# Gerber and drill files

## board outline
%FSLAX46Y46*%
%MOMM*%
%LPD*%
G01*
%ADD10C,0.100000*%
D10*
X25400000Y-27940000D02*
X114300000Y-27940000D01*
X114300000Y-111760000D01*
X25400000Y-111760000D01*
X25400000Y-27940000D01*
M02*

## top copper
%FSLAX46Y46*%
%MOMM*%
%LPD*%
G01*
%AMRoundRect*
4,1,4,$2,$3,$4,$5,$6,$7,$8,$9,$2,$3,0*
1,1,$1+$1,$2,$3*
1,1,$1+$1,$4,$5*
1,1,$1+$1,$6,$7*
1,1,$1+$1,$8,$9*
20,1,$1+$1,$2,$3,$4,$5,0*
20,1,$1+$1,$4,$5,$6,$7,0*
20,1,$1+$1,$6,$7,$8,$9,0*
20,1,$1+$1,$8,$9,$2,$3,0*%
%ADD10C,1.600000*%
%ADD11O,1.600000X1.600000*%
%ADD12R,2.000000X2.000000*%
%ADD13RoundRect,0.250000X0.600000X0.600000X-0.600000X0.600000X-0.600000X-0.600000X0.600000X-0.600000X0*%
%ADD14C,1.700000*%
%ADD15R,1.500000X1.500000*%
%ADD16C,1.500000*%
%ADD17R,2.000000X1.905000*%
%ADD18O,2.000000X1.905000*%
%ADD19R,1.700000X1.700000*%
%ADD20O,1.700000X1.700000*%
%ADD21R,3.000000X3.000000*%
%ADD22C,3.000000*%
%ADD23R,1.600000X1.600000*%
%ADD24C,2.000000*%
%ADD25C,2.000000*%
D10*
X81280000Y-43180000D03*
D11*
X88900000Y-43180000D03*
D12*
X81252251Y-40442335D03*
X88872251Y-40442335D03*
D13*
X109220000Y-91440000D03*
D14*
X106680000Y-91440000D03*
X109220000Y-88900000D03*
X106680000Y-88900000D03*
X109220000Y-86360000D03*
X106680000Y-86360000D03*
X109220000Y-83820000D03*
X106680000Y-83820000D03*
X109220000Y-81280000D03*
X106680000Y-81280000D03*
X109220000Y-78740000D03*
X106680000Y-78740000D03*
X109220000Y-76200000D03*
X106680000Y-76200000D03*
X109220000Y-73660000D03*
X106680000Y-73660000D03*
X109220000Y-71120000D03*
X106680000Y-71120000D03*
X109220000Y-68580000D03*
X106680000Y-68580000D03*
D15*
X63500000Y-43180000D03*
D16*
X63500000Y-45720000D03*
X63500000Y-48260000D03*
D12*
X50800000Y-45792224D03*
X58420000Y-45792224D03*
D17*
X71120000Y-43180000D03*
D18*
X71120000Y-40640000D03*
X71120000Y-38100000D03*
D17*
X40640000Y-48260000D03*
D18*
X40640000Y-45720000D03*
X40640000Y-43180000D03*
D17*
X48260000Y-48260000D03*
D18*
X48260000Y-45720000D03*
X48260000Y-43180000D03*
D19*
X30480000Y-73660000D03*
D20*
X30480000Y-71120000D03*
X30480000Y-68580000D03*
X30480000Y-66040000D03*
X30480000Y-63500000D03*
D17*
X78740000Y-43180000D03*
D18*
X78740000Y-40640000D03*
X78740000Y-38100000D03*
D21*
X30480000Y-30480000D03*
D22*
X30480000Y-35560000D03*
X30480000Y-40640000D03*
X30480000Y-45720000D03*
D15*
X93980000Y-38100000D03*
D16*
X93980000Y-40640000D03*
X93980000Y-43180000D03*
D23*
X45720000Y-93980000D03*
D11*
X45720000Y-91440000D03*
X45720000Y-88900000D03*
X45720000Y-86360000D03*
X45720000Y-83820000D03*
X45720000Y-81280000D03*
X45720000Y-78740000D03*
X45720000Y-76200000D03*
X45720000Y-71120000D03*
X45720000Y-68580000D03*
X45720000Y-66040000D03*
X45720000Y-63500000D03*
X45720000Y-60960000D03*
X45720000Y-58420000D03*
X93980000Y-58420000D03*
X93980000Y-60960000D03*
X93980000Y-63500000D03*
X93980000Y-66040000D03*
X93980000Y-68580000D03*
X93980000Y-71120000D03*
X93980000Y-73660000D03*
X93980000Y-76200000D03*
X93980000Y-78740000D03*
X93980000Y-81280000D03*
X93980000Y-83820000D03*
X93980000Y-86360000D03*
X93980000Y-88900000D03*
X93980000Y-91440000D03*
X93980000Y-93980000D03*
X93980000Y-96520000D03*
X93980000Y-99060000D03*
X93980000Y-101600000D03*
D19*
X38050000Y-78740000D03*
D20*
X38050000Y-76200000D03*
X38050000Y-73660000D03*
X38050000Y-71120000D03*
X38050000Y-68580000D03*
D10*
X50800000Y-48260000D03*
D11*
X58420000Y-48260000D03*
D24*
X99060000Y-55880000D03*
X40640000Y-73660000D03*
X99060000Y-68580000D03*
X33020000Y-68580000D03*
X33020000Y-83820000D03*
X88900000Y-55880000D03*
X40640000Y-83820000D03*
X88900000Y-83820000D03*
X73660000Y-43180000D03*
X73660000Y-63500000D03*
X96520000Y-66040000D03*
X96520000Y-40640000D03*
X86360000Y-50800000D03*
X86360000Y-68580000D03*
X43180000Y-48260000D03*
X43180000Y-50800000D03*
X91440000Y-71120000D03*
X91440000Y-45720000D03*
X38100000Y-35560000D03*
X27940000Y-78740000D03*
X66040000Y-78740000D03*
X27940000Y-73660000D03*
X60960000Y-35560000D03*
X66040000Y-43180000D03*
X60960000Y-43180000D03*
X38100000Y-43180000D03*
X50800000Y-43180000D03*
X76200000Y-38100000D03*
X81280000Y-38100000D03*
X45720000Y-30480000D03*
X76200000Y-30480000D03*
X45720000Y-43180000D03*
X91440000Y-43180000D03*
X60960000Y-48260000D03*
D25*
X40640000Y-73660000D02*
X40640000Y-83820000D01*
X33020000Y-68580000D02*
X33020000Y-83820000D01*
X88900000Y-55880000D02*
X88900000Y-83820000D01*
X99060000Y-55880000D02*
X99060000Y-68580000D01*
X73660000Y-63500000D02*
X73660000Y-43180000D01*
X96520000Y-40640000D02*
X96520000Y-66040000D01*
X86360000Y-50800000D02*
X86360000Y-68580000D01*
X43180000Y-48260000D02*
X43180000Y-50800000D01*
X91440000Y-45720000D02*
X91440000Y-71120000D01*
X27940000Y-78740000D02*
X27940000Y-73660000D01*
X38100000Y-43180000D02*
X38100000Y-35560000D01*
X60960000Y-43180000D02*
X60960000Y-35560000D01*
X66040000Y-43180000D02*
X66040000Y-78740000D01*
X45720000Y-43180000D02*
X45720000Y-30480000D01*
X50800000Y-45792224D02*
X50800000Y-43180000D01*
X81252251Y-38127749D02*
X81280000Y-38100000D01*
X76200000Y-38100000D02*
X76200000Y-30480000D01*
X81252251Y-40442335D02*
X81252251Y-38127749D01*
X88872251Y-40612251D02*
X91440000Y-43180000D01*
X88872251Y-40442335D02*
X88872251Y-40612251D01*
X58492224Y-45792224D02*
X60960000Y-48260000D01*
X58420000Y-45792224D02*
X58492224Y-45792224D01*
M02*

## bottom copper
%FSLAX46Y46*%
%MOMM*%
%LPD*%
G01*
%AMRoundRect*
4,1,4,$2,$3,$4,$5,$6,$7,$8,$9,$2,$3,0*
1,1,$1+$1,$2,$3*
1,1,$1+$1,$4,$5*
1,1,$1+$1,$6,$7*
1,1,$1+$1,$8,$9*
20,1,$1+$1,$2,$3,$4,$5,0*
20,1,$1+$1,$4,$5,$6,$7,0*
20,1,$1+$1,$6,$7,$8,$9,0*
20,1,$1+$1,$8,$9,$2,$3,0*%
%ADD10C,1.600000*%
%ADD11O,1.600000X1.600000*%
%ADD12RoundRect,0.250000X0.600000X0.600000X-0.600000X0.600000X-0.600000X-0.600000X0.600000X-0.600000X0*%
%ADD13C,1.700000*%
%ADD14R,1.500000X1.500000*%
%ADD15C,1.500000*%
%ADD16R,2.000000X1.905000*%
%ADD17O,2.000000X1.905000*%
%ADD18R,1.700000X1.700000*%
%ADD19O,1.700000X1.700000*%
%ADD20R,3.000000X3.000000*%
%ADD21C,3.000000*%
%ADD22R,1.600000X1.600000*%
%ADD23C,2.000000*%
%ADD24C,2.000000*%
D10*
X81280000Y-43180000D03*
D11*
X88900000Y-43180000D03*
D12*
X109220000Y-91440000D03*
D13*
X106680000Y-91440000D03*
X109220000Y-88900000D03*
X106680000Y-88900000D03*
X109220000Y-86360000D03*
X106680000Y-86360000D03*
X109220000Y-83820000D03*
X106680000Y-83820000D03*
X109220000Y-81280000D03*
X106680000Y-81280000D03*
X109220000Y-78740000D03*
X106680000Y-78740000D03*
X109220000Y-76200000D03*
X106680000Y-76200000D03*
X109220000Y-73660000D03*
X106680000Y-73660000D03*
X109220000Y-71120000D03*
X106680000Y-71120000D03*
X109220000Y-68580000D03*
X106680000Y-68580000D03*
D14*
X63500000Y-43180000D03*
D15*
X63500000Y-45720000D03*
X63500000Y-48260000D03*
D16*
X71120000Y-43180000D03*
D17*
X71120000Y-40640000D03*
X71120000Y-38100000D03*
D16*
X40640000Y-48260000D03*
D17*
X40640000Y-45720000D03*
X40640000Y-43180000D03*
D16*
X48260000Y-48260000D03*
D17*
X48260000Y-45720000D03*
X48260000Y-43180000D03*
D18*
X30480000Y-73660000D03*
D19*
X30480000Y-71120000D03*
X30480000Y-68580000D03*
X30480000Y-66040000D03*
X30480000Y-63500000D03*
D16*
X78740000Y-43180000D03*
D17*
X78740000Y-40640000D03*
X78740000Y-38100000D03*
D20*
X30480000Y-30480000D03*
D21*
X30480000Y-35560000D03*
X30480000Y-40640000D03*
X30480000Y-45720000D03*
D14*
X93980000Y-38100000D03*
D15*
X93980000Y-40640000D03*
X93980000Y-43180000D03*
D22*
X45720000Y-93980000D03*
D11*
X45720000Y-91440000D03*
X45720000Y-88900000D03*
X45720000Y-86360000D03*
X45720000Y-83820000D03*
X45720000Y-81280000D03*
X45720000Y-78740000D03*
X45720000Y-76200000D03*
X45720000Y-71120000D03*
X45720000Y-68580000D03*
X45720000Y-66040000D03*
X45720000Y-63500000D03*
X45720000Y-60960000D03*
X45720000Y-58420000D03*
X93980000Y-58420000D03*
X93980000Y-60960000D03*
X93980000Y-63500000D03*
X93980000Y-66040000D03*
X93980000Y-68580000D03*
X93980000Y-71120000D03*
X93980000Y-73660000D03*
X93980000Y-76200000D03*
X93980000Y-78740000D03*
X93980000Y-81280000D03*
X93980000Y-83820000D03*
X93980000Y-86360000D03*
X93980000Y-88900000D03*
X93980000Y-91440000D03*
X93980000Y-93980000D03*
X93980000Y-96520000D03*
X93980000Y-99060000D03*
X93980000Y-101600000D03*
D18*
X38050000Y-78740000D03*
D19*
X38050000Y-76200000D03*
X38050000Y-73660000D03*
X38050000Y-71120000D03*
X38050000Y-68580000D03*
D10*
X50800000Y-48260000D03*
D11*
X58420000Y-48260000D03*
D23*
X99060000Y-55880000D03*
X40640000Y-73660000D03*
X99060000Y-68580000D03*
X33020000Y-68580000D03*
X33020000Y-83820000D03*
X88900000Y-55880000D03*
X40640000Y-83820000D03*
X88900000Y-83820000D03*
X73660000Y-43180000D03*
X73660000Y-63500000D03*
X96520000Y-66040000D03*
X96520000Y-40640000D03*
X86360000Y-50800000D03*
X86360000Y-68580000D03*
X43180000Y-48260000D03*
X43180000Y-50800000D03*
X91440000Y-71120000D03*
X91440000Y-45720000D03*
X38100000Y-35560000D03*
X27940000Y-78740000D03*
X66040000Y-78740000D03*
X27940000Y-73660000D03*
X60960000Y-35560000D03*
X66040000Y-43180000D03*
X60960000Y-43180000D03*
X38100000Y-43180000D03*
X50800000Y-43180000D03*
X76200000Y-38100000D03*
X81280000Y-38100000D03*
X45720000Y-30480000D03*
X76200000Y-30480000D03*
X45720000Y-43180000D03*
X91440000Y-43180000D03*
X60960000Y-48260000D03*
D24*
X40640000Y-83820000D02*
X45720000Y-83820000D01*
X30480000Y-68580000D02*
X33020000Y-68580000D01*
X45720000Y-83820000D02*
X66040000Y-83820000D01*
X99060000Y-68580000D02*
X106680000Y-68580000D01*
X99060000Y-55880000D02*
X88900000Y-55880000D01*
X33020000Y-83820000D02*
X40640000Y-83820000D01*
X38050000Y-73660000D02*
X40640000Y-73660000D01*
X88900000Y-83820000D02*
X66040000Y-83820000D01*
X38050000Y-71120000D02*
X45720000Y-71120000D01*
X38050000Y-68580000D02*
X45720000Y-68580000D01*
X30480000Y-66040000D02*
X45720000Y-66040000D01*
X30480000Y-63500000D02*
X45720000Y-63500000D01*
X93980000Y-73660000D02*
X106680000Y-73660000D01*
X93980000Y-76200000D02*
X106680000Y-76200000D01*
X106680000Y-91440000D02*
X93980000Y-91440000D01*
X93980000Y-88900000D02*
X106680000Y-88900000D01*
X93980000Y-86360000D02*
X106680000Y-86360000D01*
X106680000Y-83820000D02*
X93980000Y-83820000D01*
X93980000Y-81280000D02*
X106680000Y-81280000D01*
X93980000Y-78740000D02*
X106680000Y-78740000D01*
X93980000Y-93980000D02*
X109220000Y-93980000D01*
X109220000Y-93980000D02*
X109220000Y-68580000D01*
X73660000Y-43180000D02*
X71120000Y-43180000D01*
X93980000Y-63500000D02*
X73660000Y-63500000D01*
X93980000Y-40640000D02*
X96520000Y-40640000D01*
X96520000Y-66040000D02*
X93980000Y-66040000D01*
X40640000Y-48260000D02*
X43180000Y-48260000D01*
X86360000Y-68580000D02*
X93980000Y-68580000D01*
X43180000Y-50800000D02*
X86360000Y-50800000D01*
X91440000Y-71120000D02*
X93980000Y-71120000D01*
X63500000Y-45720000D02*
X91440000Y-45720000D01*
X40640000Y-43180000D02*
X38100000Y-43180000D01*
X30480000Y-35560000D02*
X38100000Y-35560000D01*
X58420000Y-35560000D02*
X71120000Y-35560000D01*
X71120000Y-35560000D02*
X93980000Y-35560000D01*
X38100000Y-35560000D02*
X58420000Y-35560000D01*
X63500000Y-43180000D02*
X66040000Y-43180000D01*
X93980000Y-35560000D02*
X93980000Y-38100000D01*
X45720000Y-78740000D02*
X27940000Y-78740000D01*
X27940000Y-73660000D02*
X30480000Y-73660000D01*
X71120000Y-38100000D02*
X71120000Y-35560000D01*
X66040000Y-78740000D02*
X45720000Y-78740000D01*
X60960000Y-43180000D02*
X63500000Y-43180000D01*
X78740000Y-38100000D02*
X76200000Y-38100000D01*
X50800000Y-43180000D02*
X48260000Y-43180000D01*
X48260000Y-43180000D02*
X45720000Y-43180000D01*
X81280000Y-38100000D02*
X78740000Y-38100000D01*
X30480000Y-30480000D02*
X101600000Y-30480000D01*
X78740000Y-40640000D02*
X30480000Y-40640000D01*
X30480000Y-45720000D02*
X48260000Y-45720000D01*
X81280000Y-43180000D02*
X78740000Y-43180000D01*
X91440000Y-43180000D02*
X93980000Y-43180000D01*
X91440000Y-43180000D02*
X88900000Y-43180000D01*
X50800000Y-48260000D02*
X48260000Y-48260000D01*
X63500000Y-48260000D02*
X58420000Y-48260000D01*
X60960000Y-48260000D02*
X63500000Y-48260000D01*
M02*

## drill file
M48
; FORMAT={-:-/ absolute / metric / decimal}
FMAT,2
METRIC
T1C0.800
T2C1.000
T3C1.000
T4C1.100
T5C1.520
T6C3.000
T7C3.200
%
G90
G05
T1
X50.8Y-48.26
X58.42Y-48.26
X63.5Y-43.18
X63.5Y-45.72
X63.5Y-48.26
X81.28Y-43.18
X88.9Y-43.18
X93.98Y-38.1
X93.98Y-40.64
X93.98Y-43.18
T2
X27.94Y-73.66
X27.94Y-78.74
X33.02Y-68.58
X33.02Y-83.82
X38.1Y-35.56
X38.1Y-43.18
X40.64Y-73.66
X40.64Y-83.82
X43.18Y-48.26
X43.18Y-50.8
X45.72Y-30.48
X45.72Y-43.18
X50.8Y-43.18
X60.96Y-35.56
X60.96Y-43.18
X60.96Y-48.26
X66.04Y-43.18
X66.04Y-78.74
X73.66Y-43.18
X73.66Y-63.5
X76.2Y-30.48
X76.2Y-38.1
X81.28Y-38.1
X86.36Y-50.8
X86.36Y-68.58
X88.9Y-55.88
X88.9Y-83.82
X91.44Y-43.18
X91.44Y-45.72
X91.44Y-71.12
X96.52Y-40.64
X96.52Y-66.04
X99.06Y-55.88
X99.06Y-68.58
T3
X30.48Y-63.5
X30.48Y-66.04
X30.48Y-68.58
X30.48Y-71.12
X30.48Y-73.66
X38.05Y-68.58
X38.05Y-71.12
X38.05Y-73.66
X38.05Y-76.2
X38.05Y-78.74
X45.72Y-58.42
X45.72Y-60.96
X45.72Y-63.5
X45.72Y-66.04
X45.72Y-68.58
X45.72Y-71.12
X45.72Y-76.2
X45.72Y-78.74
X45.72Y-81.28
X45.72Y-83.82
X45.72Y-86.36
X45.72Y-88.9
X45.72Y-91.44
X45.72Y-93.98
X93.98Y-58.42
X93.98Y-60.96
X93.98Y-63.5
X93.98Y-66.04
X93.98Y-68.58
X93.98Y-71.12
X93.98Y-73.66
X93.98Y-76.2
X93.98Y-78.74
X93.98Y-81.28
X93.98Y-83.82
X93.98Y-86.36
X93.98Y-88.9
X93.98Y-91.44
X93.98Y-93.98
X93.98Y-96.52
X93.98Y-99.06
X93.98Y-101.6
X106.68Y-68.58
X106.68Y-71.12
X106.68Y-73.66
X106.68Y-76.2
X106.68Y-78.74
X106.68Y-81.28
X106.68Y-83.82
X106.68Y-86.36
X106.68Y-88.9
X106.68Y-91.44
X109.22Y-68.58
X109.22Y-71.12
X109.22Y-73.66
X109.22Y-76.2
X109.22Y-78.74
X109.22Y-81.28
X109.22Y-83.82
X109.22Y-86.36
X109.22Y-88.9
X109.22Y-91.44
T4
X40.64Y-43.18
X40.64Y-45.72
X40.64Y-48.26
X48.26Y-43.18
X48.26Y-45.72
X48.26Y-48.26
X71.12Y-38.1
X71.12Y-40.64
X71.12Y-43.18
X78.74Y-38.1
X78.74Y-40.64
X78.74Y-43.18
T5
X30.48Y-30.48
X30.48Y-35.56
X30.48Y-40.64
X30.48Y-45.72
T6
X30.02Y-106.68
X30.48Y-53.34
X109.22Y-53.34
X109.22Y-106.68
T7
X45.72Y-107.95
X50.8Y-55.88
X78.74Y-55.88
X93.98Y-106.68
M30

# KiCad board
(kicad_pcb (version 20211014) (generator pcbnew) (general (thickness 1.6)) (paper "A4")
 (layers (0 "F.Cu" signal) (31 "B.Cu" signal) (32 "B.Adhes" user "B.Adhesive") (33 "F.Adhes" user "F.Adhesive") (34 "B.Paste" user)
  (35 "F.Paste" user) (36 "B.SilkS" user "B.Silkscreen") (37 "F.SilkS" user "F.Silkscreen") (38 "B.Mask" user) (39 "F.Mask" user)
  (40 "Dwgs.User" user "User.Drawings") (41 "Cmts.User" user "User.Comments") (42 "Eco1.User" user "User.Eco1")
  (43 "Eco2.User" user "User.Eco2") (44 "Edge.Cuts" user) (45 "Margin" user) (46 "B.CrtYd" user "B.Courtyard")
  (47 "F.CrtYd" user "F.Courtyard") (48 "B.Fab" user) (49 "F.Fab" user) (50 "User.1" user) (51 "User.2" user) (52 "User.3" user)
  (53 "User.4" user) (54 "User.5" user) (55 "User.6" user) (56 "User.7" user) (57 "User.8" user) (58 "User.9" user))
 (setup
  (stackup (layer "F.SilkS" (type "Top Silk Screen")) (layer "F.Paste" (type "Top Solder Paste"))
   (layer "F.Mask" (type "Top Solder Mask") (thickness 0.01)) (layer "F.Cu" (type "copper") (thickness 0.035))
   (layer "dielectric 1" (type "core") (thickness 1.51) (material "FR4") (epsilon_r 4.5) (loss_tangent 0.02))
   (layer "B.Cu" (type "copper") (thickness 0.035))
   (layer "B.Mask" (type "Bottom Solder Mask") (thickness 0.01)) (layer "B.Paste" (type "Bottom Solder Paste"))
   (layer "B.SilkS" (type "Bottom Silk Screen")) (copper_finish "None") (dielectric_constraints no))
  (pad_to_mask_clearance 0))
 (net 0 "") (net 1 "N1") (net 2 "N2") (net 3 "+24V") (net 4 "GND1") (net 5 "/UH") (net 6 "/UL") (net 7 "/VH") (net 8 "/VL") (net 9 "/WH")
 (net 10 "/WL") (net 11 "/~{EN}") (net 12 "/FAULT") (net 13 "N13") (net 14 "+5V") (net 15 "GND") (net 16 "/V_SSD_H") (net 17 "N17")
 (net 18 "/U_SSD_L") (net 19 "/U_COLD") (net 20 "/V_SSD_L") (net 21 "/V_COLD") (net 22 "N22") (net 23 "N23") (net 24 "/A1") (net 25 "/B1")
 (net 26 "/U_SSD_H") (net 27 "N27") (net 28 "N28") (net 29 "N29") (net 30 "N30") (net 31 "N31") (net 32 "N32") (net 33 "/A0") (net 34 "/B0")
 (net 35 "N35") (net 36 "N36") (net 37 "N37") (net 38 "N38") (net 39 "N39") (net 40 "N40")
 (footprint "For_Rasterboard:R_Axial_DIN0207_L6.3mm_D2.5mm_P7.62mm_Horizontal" (layer "F.Cu") (at 81.28 43.18)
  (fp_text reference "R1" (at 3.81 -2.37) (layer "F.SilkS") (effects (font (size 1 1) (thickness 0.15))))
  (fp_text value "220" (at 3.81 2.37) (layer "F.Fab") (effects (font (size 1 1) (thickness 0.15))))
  (pad "1" thru_hole circle (at 0 0) (size 1.6 1.6) (drill 0.8) (layers *.Cu *.Mask) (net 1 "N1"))
  (pad "2" thru_hole oval (at 7.62 0) (size 1.6 1.6) (drill 0.8) (layers *.Cu *.Mask) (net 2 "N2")))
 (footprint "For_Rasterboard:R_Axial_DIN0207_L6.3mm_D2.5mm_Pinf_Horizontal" (layer "F.Cu") (at 81.252251 40.442335)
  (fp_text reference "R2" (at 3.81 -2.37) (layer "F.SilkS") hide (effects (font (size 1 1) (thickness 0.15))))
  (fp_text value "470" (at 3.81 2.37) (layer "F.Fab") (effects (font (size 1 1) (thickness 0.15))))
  (pad "1" smd rect locked (at 0 0) (size 2 2) (layers "F.Cu") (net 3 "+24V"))
  (pad "2" smd rect locked (at 7.62 0) (size 2 2) (layers "F.Cu") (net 2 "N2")))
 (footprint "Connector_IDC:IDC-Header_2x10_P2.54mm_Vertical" (layer "F.Cu") (at 109.22 91.44 180)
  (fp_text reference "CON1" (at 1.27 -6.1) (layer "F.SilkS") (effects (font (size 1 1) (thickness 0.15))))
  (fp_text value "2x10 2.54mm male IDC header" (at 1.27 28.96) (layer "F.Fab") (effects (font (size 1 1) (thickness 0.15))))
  (pad "1" thru_hole roundrect (at 0 0 180) (size 1.7 1.7) (drill 1) (layers *.Cu *.Mask) (roundrect_rratio 0.147059) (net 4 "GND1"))
  (pad "2" thru_hole circle (at 2.54 0 180) (size 1.7 1.7) (drill 1) (layers *.Cu *.Mask) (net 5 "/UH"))
  (pad "3" thru_hole circle (at 0 2.54 180) (size 1.7 1.7) (drill 1) (layers *.Cu *.Mask) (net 4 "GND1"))
  (pad "4" thru_hole circle (at 2.54 2.54 180) (size 1.7 1.7) (drill 1) (layers *.Cu *.Mask) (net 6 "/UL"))
  (pad "5" thru_hole circle (at 0 5.08 180) (size 1.7 1.7) (drill 1) (layers *.Cu *.Mask) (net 4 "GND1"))
  (pad "6" thru_hole circle (at 2.54 5.08 180) (size 1.7 1.7) (drill 1) (layers *.Cu *.Mask) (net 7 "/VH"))
  (pad "7" thru_hole circle (at 0 7.62 180) (size 1.7 1.7) (drill 1) (layers *.Cu *.Mask) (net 4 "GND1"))
  (pad "8" thru_hole circle (at 2.54 7.62 180) (size 1.7 1.7) (drill 1) (layers *.Cu *.Mask) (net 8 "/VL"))
  (pad "9" thru_hole circle (at 0 10.16 180) (size 1.7 1.7) (drill 1) (layers *.Cu *.Mask) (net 4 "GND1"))
  (pad "10" thru_hole circle (at 2.54 10.16 180) (size 1.7 1.7) (drill 1) (layers *.Cu *.Mask) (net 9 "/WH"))
  (pad "11" thru_hole circle (at 0 12.7 180) (size 1.7 1.7) (drill 1) (layers *.Cu *.Mask) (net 4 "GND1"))
  (pad "12" thru_hole circle (at 2.54 12.7 180) (size 1.7 1.7) (drill 1) (layers *.Cu *.Mask) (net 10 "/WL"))
  (pad "13" thru_hole circle (at 0 15.24 180) (size 1.7 1.7) (drill 1) (layers *.Cu *.Mask) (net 4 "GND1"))
  (pad "14" thru_hole circle (at 2.54 15.24 180) (size 1.7 1.7) (drill 1) (layers *.Cu *.Mask) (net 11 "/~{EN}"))
  (pad "15" thru_hole circle (at 0 17.78 180) (size 1.7 1.7) (drill 1) (layers *.Cu *.Mask) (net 4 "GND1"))
  (pad "16" thru_hole circle (at 2.54 17.78 180) (size 1.7 1.7) (drill 1) (layers *.Cu *.Mask) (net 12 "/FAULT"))
  (pad "17" thru_hole circle (at 0 20.32 180) (size 1.7 1.7) (drill 1) (layers *.Cu *.Mask) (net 4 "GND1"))
  (pad "18" thru_hole circle (at 2.54 20.32 180) (size 1.7 1.7) (drill 1) (layers *.Cu *.Mask) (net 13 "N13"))
  (pad "19" thru_hole circle (at 0 22.86 180) (size 1.7 1.7) (drill 1) (layers *.Cu *.Mask) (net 4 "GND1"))
  (pad "20" thru_hole circle (at 2.54 22.86 180) (size 1.7 1.7) (drill 1) (layers *.Cu *.Mask) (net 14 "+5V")))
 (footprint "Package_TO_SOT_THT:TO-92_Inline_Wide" (layer "F.Cu") (at 63.5 43.18 -90)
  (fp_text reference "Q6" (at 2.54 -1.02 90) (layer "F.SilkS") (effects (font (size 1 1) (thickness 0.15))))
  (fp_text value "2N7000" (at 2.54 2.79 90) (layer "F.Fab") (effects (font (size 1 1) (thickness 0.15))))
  (pad "1" thru_hole rect (at 0 0 270) (size 1.5 1.5) (drill 0.8) (layers *.Cu *.Mask) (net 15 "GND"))
  (pad "2" thru_hole circle (at 2.54 0 270) (size 1.5 1.5) (drill 0.8) (layers *.Cu *.Mask) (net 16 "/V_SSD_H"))
  (pad "3" thru_hole circle (at 5.08 0 270) (size 1.5 1.5) (drill 0.8) (layers *.Cu *.Mask) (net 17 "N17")))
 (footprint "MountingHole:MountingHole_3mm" (layer "F.Cu") (at 30.02 106.68)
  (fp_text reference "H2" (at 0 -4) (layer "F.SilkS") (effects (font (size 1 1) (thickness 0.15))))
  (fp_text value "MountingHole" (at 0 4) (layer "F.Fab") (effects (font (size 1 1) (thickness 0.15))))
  (pad "" np_thru_hole circle (at 0 0) (size 3 3) (drill 3) (layers *.Cu *.Mask)))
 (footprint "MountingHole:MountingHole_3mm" (layer "F.Cu") (at 109.22 53.34)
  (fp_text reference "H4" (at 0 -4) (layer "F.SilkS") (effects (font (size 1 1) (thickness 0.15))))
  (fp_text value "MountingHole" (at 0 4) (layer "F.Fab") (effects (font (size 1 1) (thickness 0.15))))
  (pad "" np_thru_hole circle (at 0 0) (size 3 3) (drill 3) (layers *.Cu *.Mask)))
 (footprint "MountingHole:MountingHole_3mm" (layer "F.Cu") (at 109.22 106.68)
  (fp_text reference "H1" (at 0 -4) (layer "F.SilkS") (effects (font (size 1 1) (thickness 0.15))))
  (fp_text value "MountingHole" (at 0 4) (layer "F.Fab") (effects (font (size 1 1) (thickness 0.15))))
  (pad "" np_thru_hole circle (at 0 0) (size 3 3) (drill 3) (layers *.Cu *.Mask)))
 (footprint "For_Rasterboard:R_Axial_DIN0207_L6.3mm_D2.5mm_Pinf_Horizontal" (layer "F.Cu") (at 50.8 45.792224)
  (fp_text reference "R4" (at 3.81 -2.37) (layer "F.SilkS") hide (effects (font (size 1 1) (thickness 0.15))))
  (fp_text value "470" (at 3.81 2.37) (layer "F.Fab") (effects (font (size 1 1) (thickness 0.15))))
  (pad "1" smd rect locked (at 0 0) (size 2 2) (layers "F.Cu") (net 3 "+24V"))
  (pad "2" smd rect locked (at 7.62 0) (size 2 2) (layers "F.Cu") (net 17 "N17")))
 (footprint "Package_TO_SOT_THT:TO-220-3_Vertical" (layer "F.Cu") (at 71.12 43.18 90)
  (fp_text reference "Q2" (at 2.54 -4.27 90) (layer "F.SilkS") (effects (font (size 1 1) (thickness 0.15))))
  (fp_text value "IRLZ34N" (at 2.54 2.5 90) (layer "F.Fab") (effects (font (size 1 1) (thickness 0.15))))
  (pad "1" thru_hole rect (at 0 0 90) (size 1.905 2) (drill 1.1) (layers *.Cu *.Mask) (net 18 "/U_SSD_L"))
  (pad "2" thru_hole oval (at 2.54 0 90) (size 1.905 2) (drill 1.1) (layers *.Cu *.Mask) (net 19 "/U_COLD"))
  (pad "3" thru_hole oval (at 5.08 0 90) (size 1.905 2) (drill 1.1) (layers *.Cu *.Mask) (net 15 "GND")))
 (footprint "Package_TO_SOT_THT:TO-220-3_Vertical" (layer "F.Cu") (at 40.64 48.26 90)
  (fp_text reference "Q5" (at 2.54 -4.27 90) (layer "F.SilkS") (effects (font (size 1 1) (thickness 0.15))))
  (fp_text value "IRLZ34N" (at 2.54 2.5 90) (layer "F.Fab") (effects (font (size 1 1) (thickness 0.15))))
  (pad "1" thru_hole rect (at 0 0 90) (size 1.905 2) (drill 1.1) (layers *.Cu *.Mask) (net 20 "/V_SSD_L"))
  (pad "2" thru_hole oval (at 2.54 0 90) (size 1.905 2) (drill 1.1) (layers *.Cu *.Mask) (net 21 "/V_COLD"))
  (pad "3" thru_hole oval (at 5.08 0 90) (size 1.905 2) (drill 1.1) (layers *.Cu *.Mask) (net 15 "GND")))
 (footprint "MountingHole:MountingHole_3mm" (layer "F.Cu") (at 30.48 53.34)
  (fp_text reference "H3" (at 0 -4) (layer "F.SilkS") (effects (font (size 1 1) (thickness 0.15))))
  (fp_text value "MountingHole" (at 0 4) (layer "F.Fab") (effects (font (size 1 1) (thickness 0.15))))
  (pad "" np_thru_hole circle (at 0 0) (size 3 3) (drill 3) (layers *.Cu *.Mask)))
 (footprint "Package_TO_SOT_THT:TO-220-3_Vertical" (layer "F.Cu") (at 48.26 48.26 90)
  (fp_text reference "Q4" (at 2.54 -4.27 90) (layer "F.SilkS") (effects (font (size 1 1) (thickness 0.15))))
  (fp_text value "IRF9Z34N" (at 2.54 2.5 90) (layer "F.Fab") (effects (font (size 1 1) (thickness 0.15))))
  (pad "1" thru_hole rect (at 0 0 90) (size 1.905 2) (drill 1.1) (layers *.Cu *.Mask) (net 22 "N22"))
  (pad "2" thru_hole oval (at 2.54 0 90) (size 1.905 2) (drill 1.1) (layers *.Cu *.Mask) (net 21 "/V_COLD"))
  (pad "3" thru_hole oval (at 5.08 0 90) (size 1.905 2) (drill 1.1) (layers *.Cu *.Mask) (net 3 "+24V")))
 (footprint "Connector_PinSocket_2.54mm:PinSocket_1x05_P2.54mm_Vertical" (layer "F.Cu") (at 30.48 73.66 180)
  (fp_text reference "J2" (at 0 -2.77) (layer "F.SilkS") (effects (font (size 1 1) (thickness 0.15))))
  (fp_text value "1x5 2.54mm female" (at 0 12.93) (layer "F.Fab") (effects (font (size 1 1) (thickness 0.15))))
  (pad "1" thru_hole rect (at 0 0 180) (size 1.7 1.7) (drill 1) (layers *.Cu *.Mask) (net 15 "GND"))
  (pad "2" thru_hole oval (at 0 2.54 180) (size 1.7 1.7) (drill 1) (layers *.Cu *.Mask) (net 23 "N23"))
  (pad "3" thru_hole oval (at 0 5.08 180) (size 1.7 1.7) (drill 1) (layers *.Cu *.Mask) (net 14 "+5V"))
  (pad "4" thru_hole oval (at 0 7.62 180) (size 1.7 1.7) (drill 1) (layers *.Cu *.Mask) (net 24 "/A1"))
  (pad "5" thru_hole oval (at 0 10.16 180) (size 1.7 1.7) (drill 1) (layers *.Cu *.Mask) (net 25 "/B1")))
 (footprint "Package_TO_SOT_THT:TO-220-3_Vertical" (layer "F.Cu") (at 78.74 43.18 90)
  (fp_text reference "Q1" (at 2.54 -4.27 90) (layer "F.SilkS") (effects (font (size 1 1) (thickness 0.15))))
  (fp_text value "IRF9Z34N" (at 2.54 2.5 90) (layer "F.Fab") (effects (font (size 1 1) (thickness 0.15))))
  (pad "1" thru_hole rect (at 0 0 90) (size 1.905 2) (drill 1.1) (layers *.Cu *.Mask) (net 1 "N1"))
  (pad "2" thru_hole oval (at 2.54 0 90) (size 1.905 2) (drill 1.1) (layers *.Cu *.Mask) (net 19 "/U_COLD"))
  (pad "3" thru_hole oval (at 5.08 0 90) (size 1.905 2) (drill 1.1) (layers *.Cu *.Mask) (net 3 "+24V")))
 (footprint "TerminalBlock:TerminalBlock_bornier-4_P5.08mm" (layer "F.Cu") (at 30.48 30.48 -90)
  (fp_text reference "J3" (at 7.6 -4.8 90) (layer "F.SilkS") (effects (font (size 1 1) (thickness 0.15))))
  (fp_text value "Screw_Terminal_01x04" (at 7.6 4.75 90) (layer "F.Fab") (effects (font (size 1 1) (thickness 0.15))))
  (pad "1" thru_hole rect (at 0 0 270) (size 3 3) (drill 1.52) (layers *.Cu *.Mask) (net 3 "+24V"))
  (pad "2" thru_hole circle (at 5.08 0 270) (size 3 3) (drill 1.52) (layers *.Cu *.Mask) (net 15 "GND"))
  (pad "3" thru_hole circle (at 10.16 0 270) (size 3 3) (drill 1.52) (layers *.Cu *.Mask) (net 19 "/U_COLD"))
  (pad "4" thru_hole circle (at 15.24 0 270) (size 3 3) (drill 1.52) (layers *.Cu *.Mask) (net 21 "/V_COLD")))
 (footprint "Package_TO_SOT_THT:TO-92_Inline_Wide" (layer "F.Cu") (at 93.98 38.1 -90)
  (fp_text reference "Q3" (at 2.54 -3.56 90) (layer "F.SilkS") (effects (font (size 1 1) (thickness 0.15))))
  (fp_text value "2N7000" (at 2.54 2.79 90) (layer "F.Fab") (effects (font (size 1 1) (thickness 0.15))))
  (pad "1" thru_hole rect (at 0 0 270) (size 1.5 1.5) (drill 0.8) (layers *.Cu *.Mask) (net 15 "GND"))
  (pad "2" thru_hole circle (at 2.54 0 270) (size 1.5 1.5) (drill 0.8) (layers *.Cu *.Mask) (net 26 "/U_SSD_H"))
  (pad "3" thru_hole circle (at 5.08 0 270) (size 1.5 1.5) (drill 0.8) (layers *.Cu *.Mask) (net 2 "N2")))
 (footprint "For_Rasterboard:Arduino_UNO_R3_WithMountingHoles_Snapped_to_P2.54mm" (layer "F.Cu") (at 45.72 93.98 90)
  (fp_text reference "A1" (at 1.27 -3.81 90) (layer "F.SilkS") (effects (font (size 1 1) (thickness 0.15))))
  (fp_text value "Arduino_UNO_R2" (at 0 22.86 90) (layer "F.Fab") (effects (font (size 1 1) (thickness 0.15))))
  (pad "" np_thru_hole circle (at -13.97 0 180) (size 3.2 3.2) (drill 3.2) (layers *.Cu *.Mask))
  (pad "" np_thru_hole circle (at 38.1 5.08 180) (size 3.2 3.2) (drill 3.2) (layers *.Cu *.Mask))
  (pad "" np_thru_hole circle (at -12.7 48.26 180) (size 3.2 3.2) (drill 3.2) (layers *.Cu *.Mask))
  (pad "" np_thru_hole circle (at 38.1 33.02 180) (size 3.2 3.2) (drill 3.2) (layers *.Cu *.Mask))
  (pad "1" thru_hole rect (at 0 0 180) (size 1.6 1.6) (drill 1) (layers *.Cu *.Mask) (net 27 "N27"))
  (pad "2" thru_hole oval (at 2.54 0 180) (size 1.6 1.6) (drill 1) (layers *.Cu *.Mask) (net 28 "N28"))
  (pad "3" thru_hole oval (at 5.08 0 180) (size 1.6 1.6) (drill 1) (layers *.Cu *.Mask) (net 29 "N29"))
  (pad "4" thru_hole oval (at 7.62 0 180) (size 1.6 1.6) (drill 1) (layers *.Cu *.Mask) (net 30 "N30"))
  (pad "5" thru_hole oval (at 10.16 0 180) (size 1.6 1.6) (drill 1) (layers *.Cu *.Mask) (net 14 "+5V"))
  (pad "6" thru_hole oval (at 12.7 0 180) (size 1.6 1.6) (drill 1) (layers *.Cu *.Mask) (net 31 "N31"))
  (pad "7" thru_hole oval (at 15.24 0 180) (size 1.6 1.6) (drill 1) (layers *.Cu *.Mask) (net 15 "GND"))
  (pad "8" thru_hole oval (at 17.78 0 180) (size 1.6 1.6) (drill 1) (layers *.Cu *.Mask) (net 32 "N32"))
  (pad "9" thru_hole oval (at 22.86 0 180) (size 1.6 1.6) (drill 1) (layers *.Cu *.Mask) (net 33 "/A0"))
  (pad "10" thru_hole oval (at 25.4 0 180) (size 1.6 1.6) (drill 1) (layers *.Cu *.Mask) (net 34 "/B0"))
  (pad "11" thru_hole oval (at 27.94 0 180) (size 1.6 1.6) (drill 1) (layers *.Cu *.Mask) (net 24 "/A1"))
  (pad "12" thru_hole oval (at 30.48 0 180) (size 1.6 1.6) (drill 1) (layers *.Cu *.Mask) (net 25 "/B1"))
  (pad "13" thru_hole oval (at 33.02 0 180) (size 1.6 1.6) (drill 1) (layers *.Cu *.Mask) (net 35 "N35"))
  (pad "14" thru_hole oval (at 35.56 0 180) (size 1.6 1.6) (drill 1) (layers *.Cu *.Mask) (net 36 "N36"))
  (pad "15" thru_hole oval (at 35.56 48.26 180) (size 1.6 1.6) (drill 1) (layers *.Cu *.Mask) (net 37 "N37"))
  (pad "16" thru_hole oval (at 33.02 48.26 180) (size 1.6 1.6) (drill 1) (layers *.Cu *.Mask) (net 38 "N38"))
  (pad "17" thru_hole oval (at 30.48 48.26 180) (size 1.6 1.6) (drill 1) (layers *.Cu *.Mask) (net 18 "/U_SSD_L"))
  (pad "18" thru_hole oval (at 27.94 48.26 180) (size 1.6 1.6) (drill 1) (layers *.Cu *.Mask) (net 26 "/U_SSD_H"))
  (pad "19" thru_hole oval (at 25.4 48.26 180) (size 1.6 1.6) (drill 1) (layers *.Cu *.Mask) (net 20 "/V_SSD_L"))
  (pad "20" thru_hole oval (at 22.86 48.26 180) (size 1.6 1.6) (drill 1) (layers *.Cu *.Mask) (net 16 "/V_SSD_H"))
  (pad "21" thru_hole oval (at 20.32 48.26 180) (size 1.6 1.6) (drill 1) (layers *.Cu *.Mask) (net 12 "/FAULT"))
  (pad "22" thru_hole oval (at 17.78 48.26 180) (size 1.6 1.6) (drill 1) (layers *.Cu *.Mask) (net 11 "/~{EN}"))
  (pad "23" thru_hole oval (at 15.24 48.26 180) (size 1.6 1.6) (drill 1) (layers *.Cu *.Mask) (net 10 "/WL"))
  (pad "24" thru_hole oval (at 12.7 48.26 180) (size 1.6 1.6) (drill 1) (layers *.Cu *.Mask) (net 9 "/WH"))
  (pad "25" thru_hole oval (at 10.16 48.26 180) (size 1.6 1.6) (drill 1) (layers *.Cu *.Mask) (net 8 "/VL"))
  (pad "26" thru_hole oval (at 7.62 48.26 180) (size 1.6 1.6) (drill 1) (layers *.Cu *.Mask) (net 7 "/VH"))
  (pad "27" thru_hole oval (at 5.08 48.26 180) (size 1.6 1.6) (drill 1) (layers *.Cu *.Mask) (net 6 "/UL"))
  (pad "28" thru_hole oval (at 2.54 48.26 180) (size 1.6 1.6) (drill 1) (layers *.Cu *.Mask) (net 5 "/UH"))
  (pad "29" thru_hole oval (at 0 48.26 180) (size 1.6 1.6) (drill 1) (layers *.Cu *.Mask) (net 4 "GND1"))
  (pad "30" thru_hole oval (at -2.54 48.26 180) (size 1.6 1.6) (drill 1) (layers *.Cu *.Mask) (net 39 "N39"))
  (pad "31" thru_hole oval (at -5.08 48.26 180) (size 1.6 1.6) (drill 1) (layers *.Cu *.Mask))
  (pad "32" thru_hole oval (at -7.62 48.26 180) (size 1.6 1.6) (drill 1) (layers *.Cu *.Mask)))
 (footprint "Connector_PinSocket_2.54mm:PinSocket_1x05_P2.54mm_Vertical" (layer "F.Cu") (at 38.05 78.74 180)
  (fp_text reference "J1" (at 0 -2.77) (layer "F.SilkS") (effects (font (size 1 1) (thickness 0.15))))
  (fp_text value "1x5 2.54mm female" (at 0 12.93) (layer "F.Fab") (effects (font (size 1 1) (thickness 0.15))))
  (pad "1" thru_hole rect (at 0 0 180) (size 1.7 1.7) (drill 1) (layers *.Cu *.Mask) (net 15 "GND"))
  (pad "2" thru_hole oval (at 0 2.54 180) (size 1.7 1.7) (drill 1) (layers *.Cu *.Mask) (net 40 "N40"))
  (pad "3" thru_hole oval (at 0 5.08 180) (size 1.7 1.7) (drill 1) (layers *.Cu *.Mask) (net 14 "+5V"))
  (pad "4" thru_hole oval (at 0 7.62 180) (size 1.7 1.7) (drill 1) (layers *.Cu *.Mask) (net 33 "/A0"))
  (pad "5" thru_hole oval (at 0 10.16 180) (size 1.7 1.7) (drill 1) (layers *.Cu *.Mask) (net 34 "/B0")))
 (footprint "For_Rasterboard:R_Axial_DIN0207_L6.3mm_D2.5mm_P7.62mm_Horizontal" (layer "F.Cu") (at 50.8 48.26)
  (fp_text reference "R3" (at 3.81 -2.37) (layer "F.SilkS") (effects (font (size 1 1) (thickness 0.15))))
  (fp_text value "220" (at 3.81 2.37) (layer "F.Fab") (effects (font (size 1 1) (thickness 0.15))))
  (pad "1" thru_hole circle (at 0 0) (size 1.6 1.6) (drill 0.8) (layers *.Cu *.Mask) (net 22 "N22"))
  (pad "2" thru_hole oval (at 7.62 0) (size 1.6 1.6) (drill 0.8) (layers *.Cu *.Mask) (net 17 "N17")))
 (gr_rect (start 114.3 27.94) (end 25.4 111.76) (layer "Edge.Cuts") (width 0.1) (fill none))
 (segment (start 40.64 73.66) (end 40.64 83.82) (width 2) (layer "F.Cu") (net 14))
 (segment (start 33.02 68.58) (end 33.02 83.82) (width 2) (layer "F.Cu") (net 14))
 (segment (start 88.9 55.88) (end 88.9 83.82) (width 2) (layer "F.Cu") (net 14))
 (segment (start 99.06 55.88) (end 99.06 68.58) (width 2) (layer "F.Cu") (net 14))
 (via (at 99.06 55.88) (size 2) (drill 1) (layers "F.Cu" "B.Cu") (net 14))
 (via (at 40.64 73.66) (size 2) (drill 1) (layers "F.Cu" "B.Cu") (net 14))
 (via (at 99.06 68.58) (size 2) (drill 1) (layers "F.Cu" "B.Cu") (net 14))
 (via (at 33.02 68.58) (size 2) (drill 1) (layers "F.Cu" "B.Cu") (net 14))
 (via (at 33.02 83.82) (size 2) (drill 1) (layers "F.Cu" "B.Cu") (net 14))
 (via (at 88.9 55.88) (size 2) (drill 1) (layers "F.Cu" "B.Cu") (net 14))
 (via (at 40.64 83.82) (size 2) (drill 1) (layers "F.Cu" "B.Cu") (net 14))
 (via (at 88.9 83.82) (size 2) (drill 1) (layers "F.Cu" "B.Cu") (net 14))
 (segment (start 40.64 83.82) (end 45.72 83.82) (width 2) (layer "B.Cu") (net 14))
 (segment (start 30.48 68.58) (end 33.02 68.58) (width 2) (layer "B.Cu") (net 14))
 (segment (start 45.72 83.82) (end 66.04 83.82) (width 2) (layer "B.Cu") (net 14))
 (segment (start 99.06 68.58) (end 106.68 68.58) (width 2) (layer "B.Cu") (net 14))
 (segment (start 99.06 55.88) (end 88.9 55.88) (width 2) (layer "B.Cu") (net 14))
 (segment (start 33.02 83.82) (end 40.64 83.82) (width 2) (layer "B.Cu") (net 14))
 (segment (start 38.05 73.66) (end 40.64 73.66) (width 2) (layer "B.Cu") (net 14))
 (segment (start 88.9 83.82) (end 66.04 83.82) (width 2) (layer "B.Cu") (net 14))
 (segment (start 38.05 71.12) (end 45.72 71.12) (width 2) (layer "B.Cu") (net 33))
 (segment (start 38.05 68.58) (end 45.72 68.58) (width 2) (layer "B.Cu") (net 34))
 (segment (start 30.48 66.04) (end 45.72 66.04) (width 2) (layer "B.Cu") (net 24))
 (segment (start 30.48 63.5) (end 45.72 63.5) (width 2) (layer "B.Cu") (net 25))
 (segment (start 93.98 73.66) (end 106.68 73.66) (width 2) (layer "B.Cu") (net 12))
 (segment (start 93.98 76.2) (end 106.68 76.2) (width 2) (layer "B.Cu") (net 11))
 (segment (start 106.68 91.44) (end 93.98 91.44) (width 2) (layer "B.Cu") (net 5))
 (segment (start 93.98 88.9) (end 106.68 88.9) (width 2) (layer "B.Cu") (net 6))
 (segment (start 93.98 86.36) (end 106.68 86.36) (width 2) (layer "B.Cu") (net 7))
 (segment (start 106.68 83.82) (end 93.98 83.82) (width 2) (layer "B.Cu") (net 8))
 (segment (start 93.98 81.28) (end 106.68 81.28) (width 2) (layer "B.Cu") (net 9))
 (segment (start 93.98 78.74) (end 106.68 78.74) (width 2) (layer "B.Cu") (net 10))
 (segment (start 93.98 93.98) (end 109.22 93.98) (width 2) (layer "B.Cu") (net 4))
 (segment (start 109.22 93.98) (end 109.22 68.58) (width 2) (layer "B.Cu") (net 4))
 (segment (start 73.66 63.5) (end 73.66 43.18) (width 2) (layer "F.Cu") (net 18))
 (via (at 73.66 43.18) (size 2) (drill 1) (layers "F.Cu" "B.Cu") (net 18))
 (via (at 73.66 63.5) (size 2) (drill 1) (layers "F.Cu" "B.Cu") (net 18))
 (segment (start 73.66 43.18) (end 71.12 43.18) (width 2) (layer "B.Cu") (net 18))
 (segment (start 93.98 63.5) (end 73.66 63.5) (width 2) (layer "B.Cu") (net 18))
 (segment (start 96.52 40.64) (end 96.52 66.04) (width 2) (layer "F.Cu") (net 26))
 (via (at 96.52 66.04) (size 2) (drill 1) (layers "F.Cu" "B.Cu") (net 26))
 (via (at 96.52 40.64) (size 2) (drill 1) (layers "F.Cu" "B.Cu") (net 26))
 (segment (start 93.98 40.64) (end 96.52 40.64) (width 2) (layer "B.Cu") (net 26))
 (segment (start 96.52 66.04) (end 93.98 66.04) (width 2) (layer "B.Cu") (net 26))
 (segment (start 86.36 50.8) (end 86.36 68.58) (width 2) (layer "F.Cu") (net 20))
 (segment (start 43.18 48.26) (end 43.18 50.8) (width 2) (layer "F.Cu") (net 20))
 (via (at 86.36 50.8) (size 2) (drill 1) (layers "F.Cu" "B.Cu") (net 20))
 (via (at 86.36 68.58) (size 2) (drill 1) (layers "F.Cu" "B.Cu") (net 20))
 (via (at 43.18 48.26) (size 2) (drill 1) (layers "F.Cu" "B.Cu") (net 20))
 (via (at 43.18 50.8) (size 2) (drill 1) (layers "F.Cu" "B.Cu") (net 20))
 (segment (start 40.64 48.26) (end 43.18 48.26) (width 2) (layer "B.Cu") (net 20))
 (segment (start 86.36 68.58) (end 93.98 68.58) (width 2) (layer "B.Cu") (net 20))
 (segment (start 43.18 50.8) (end 86.36 50.8) (width 2) (layer "B.Cu") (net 20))
 (segment (start 91.44 45.72) (end 91.44 71.12) (width 2) (layer "F.Cu") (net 16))
 (via (at 91.44 71.12) (size 2) (drill 1) (layers "F.Cu" "B.Cu") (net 16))
 (via (at 91.44 45.72) (size 2) (drill 1) (layers "F.Cu" "B.Cu") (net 16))
 (segment (start 91.44 71.12) (end 93.98 71.12) (width 2) (layer "B.Cu") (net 16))
 (segment (start 63.5 45.72) (end 91.44 45.72) (width 2) (layer "B.Cu") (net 16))
 (segment (start 27.94 78.74) (end 27.94 73.66) (width 2) (layer "F.Cu") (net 15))
 (segment (start 38.1 43.18) (end 38.1 35.56) (width 2) (layer "F.Cu") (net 15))
 (segment (start 60.96 43.18) (end 60.96 35.56) (width 2) (layer "F.Cu") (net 15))
 (segment (start 66.04 43.18) (end 66.04 78.74) (width 2) (layer "F.Cu") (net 15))
 (via (at 38.1 35.56) (size 2) (drill 1) (layers "F.Cu" "B.Cu") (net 15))
 (via (at 27.94 78.74) (size 2) (drill 1) (layers "F.Cu" "B.Cu") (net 15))
 (via (at 66.04 78.74) (size 2) (drill 1) (layers "F.Cu" "B.Cu") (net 15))
 (via (at 27.94 73.66) (size 2) (drill 1) (layers "F.Cu" "B.Cu") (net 15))
 (via (at 60.96 35.56) (size 2) (drill 1) (layers "F.Cu" "B.Cu") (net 15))
 (via (at 66.04 43.18) (size 2) (drill 1) (layers "F.Cu" "B.Cu") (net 15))
 (via (at 60.96 43.18) (size 2) (drill 1) (layers "F.Cu" "B.Cu") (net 15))
 (via (at 38.1 43.18) (size 2) (drill 1) (layers "F.Cu" "B.Cu") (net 15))
 (segment (start 40.64 43.18) (end 38.1 43.18) (width 2) (layer "B.Cu") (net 15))
 (segment (start 30.48 35.56) (end 38.1 35.56) (width 2) (layer "B.Cu") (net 15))
 (segment (start 58.42 35.56) (end 71.12 35.56) (width 2) (layer "B.Cu") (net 15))
 (segment (start 71.12 35.56) (end 93.98 35.56) (width 2) (layer "B.Cu") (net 15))
 (segment (start 38.1 35.56) (end 58.42 35.56) (width 2) (layer "B.Cu") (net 15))
 (segment (start 63.5 43.18) (end 66.04 43.18) (width 2) (layer "B.Cu") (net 15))
 (segment (start 93.98 35.56) (end 93.98 38.1) (width 2) (layer "B.Cu") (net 15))
 (segment (start 45.72 78.74) (end 27.94 78.74) (width 2) (layer "B.Cu") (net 15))
 (segment (start 27.94 73.66) (end 30.48 73.66) (width 2) (layer "B.Cu") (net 15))
 (segment (start 71.12 38.1) (end 71.12 35.56) (width 2) (layer "B.Cu") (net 15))
 (segment (start 66.04 78.74) (end 45.72 78.74) (width 2) (layer "B.Cu") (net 15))
 (segment (start 60.96 43.18) (end 63.5 43.18) (width 2) (layer "B.Cu") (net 15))
 (segment (start 45.72 43.18) (end 45.72 30.48) (width 2) (layer "F.Cu") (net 3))
 (segment (start 50.8 45.792224) (end 50.8 43.18) (width 2) (layer "F.Cu") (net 3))
 (segment (start 81.252251 38.127749) (end 81.28 38.1) (width 2) (layer "F.Cu") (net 3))
 (segment (start 76.2 38.1) (end 76.2 30.48) (width 2) (layer "F.Cu") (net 3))
 (segment (start 81.252251 40.442335) (end 81.252251 38.127749) (width 2) (layer "F.Cu") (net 3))
 (via (at 50.8 43.18) (size 2) (drill 1) (layers "F.Cu" "B.Cu") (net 3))
 (via (at 76.2 38.1) (size 2) (drill 1) (layers "F.Cu" "B.Cu") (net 3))
 (via (at 81.28 38.1) (size 2) (drill 1) (layers "F.Cu" "B.Cu") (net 3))
 (via (at 45.72 30.48) (size 2) (drill 1) (layers "F.Cu" "B.Cu") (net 3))
 (via (at 76.2 30.48) (size 2) (drill 1) (layers "F.Cu" "B.Cu") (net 3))
 (via (at 45.72 43.18) (size 2) (drill 1) (layers "F.Cu" "B.Cu") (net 3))
 (segment (start 78.74 38.1) (end 76.2 38.1) (width 2) (layer "B.Cu") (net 3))
 (segment (start 50.8 43.18) (end 48.26 43.18) (width 2) (layer "B.Cu") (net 3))
 (segment (start 48.26 43.18) (end 45.72 43.18) (width 2) (layer "B.Cu") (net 3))
 (segment (start 81.28 38.1) (end 78.74 38.1) (width 2) (layer "B.Cu") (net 3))
 (segment (start 30.48 30.48) (end 101.6 30.48) (width 2) (layer "B.Cu") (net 3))
 (segment (start 78.74 40.64) (end 30.48 40.64) (width 2) (layer "B.Cu") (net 19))
 (segment (start 30.48 45.72) (end 48.26 45.72) (width 2) (layer "B.Cu") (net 21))
 (segment (start 81.28 43.18) (end 78.74 43.18) (width 2) (layer "B.Cu") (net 1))
 (segment (start 88.872251 40.612251) (end 91.44 43.18) (width 2) (layer "F.Cu") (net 2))
 (segment (start 88.872251 40.442335) (end 88.872251 40.612251) (width 2) (layer "F.Cu") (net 2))
 (via (at 91.44 43.18) (size 2) (drill 1) (layers "F.Cu" "B.Cu") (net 2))
 (segment (start 91.44 43.18) (end 93.98 43.18) (width 2) (layer "B.Cu") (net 2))
 (segment (start 91.44 43.18) (end 88.9 43.18) (width 2) (layer "B.Cu") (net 2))
 (segment (start 50.8 48.26) (end 48.26 48.26) (width 2) (layer "B.Cu") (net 22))
 (segment (start 58.492224 45.792224) (end 60.96 48.26) (width 2) (layer "F.Cu") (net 17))
 (segment (start 58.42 45.792224) (end 58.492224 45.792224) (width 2) (layer "F.Cu") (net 17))
 (via (at 60.96 48.26) (size 2) (drill 1) (layers "F.Cu" "B.Cu") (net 17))
 (segment (start 63.5 48.26) (end 58.42 48.26) (width 2) (layer "B.Cu") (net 17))
 (segment (start 60.96 48.26) (end 63.5 48.26) (width 2) (layer "B.Cu") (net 17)))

